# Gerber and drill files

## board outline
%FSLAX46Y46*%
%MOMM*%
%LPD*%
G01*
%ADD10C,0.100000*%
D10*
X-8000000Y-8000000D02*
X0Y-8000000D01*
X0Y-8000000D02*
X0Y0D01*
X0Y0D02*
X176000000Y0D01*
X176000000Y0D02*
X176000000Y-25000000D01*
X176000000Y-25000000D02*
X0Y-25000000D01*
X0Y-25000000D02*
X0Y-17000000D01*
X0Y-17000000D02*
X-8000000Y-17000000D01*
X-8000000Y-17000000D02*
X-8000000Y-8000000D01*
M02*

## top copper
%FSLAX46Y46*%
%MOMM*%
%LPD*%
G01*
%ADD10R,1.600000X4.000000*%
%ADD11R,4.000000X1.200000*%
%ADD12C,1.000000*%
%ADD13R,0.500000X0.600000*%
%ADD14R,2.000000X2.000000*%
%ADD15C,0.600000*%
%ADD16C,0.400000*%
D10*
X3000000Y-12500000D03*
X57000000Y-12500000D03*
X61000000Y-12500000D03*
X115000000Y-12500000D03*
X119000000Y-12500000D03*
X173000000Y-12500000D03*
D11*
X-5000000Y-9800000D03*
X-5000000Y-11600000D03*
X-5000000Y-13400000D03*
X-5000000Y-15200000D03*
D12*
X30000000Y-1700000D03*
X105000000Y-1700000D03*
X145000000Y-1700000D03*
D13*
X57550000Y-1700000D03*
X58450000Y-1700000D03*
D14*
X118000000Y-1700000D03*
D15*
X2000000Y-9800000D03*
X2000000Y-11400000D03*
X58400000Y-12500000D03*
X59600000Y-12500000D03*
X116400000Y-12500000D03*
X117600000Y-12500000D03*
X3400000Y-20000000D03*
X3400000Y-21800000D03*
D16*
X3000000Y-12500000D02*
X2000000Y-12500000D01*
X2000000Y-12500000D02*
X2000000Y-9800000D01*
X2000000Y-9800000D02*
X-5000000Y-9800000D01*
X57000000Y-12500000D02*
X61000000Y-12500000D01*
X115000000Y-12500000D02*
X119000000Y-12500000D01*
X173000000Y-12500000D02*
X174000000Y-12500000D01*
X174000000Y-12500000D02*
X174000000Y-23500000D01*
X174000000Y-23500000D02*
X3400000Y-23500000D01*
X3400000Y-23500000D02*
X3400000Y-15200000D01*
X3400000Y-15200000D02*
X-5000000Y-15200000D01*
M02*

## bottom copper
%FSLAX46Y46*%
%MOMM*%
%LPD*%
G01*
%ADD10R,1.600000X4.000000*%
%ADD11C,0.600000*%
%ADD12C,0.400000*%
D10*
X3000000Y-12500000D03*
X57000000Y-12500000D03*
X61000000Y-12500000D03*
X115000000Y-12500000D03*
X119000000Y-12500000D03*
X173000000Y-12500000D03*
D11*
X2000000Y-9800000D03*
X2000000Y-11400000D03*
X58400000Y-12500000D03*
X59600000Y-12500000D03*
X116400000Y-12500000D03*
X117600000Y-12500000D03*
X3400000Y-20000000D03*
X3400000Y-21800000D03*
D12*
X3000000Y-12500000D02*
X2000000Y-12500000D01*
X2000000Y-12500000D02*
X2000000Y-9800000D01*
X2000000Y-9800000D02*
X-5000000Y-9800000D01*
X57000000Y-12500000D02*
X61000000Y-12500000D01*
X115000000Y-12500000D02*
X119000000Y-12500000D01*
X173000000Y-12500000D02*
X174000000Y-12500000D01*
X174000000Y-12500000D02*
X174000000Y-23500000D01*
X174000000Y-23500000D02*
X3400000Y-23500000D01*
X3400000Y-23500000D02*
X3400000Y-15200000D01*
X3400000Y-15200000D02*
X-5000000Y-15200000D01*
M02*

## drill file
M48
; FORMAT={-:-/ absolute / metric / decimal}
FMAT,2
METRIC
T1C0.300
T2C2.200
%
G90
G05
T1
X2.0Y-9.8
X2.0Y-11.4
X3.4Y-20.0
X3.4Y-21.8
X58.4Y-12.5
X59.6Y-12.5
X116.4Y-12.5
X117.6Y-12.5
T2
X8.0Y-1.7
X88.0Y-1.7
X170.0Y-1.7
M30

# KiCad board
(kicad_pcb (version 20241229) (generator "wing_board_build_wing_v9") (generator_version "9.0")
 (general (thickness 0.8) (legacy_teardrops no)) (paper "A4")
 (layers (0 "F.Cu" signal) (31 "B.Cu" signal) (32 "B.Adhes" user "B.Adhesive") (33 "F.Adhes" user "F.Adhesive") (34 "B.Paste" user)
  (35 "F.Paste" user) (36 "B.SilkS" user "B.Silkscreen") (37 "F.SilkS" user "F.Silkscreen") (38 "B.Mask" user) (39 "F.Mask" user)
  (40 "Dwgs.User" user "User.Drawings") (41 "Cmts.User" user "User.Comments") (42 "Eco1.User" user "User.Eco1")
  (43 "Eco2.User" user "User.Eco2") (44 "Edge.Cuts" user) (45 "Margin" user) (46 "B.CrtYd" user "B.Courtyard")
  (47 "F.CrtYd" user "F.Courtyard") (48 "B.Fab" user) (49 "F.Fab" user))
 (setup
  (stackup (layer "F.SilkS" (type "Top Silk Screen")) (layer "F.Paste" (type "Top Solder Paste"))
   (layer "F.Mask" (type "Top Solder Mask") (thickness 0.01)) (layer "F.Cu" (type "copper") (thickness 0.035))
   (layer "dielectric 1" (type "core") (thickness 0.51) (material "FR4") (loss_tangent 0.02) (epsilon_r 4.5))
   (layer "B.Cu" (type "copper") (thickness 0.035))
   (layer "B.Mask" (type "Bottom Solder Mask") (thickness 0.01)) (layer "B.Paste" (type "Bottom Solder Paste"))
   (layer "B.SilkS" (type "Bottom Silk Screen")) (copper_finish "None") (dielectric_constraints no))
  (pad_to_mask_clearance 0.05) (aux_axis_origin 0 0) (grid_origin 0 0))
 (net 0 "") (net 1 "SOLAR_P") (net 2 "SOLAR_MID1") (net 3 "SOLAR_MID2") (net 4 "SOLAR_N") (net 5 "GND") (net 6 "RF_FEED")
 (gr_line (start -8 8) (end 0 8) (stroke (width 0.1) (type default)) (layer "Edge.Cuts"))
 (gr_line (start 0 8) (end 0 0) (stroke (width 0.1) (type default)) (layer "Edge.Cuts"))
 (gr_line (start 0 0) (end 176 0) (stroke (width 0.1) (type default)) (layer "Edge.Cuts"))
 (gr_line (start 176 0) (end 176 25) (stroke (width 0.1) (type default)) (layer "Edge.Cuts"))
 (gr_line (start 176 25) (end 0 25) (stroke (width 0.1) (type default)) (layer "Edge.Cuts"))
 (gr_line (start 0 25) (end 0 17) (stroke (width 0.1) (type default)) (layer "Edge.Cuts"))
 (gr_line (start 0 17) (end -8 17) (stroke (width 0.1) (type default)) (layer "Edge.Cuts"))
 (gr_line (start -8 17) (end -8 8) (stroke (width 0.1) (type default)) (layer "Edge.Cuts"))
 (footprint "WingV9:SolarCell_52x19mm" (layer "F.Cu") (at 30 12.5)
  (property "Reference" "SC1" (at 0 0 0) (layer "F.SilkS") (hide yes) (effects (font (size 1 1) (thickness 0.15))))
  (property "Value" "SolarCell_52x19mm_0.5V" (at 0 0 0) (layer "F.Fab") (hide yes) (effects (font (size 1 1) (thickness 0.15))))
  (pad "1" smd rect (at -27 0) (size 1.6 4) (layers "F.Cu" "F.Paste" "F.Mask") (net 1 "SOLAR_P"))
  (pad "2" smd rect (at 27 0) (size 1.6 4) (layers "F.Cu" "F.Paste" "F.Mask") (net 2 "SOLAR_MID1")))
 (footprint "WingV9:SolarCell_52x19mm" (layer "F.Cu") (at 88 12.5)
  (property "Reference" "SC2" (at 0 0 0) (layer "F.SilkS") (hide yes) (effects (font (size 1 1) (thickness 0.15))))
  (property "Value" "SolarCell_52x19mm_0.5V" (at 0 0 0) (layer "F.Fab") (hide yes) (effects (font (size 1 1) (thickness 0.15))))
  (pad "1" smd rect (at -27 0) (size 1.6 4) (layers "F.Cu" "F.Paste" "F.Mask") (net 2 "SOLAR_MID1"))
  (pad "2" smd rect (at 27 0) (size 1.6 4) (layers "F.Cu" "F.Paste" "F.Mask") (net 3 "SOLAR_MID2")))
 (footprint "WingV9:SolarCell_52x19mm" (layer "F.Cu") (at 146 12.5)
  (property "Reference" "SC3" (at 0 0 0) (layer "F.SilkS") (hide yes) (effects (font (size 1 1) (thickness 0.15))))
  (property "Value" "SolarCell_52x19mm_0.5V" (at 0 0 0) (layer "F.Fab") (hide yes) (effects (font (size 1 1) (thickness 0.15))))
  (pad "1" smd rect (at -27 0) (size 1.6 4) (layers "F.Cu" "F.Paste" "F.Mask") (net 3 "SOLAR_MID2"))
  (pad "2" smd rect (at 27 0) (size 1.6 4) (layers "F.Cu" "F.Paste" "F.Mask") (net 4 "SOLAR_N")))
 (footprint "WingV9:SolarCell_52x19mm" (layer "B.Cu") (at 30 12.5)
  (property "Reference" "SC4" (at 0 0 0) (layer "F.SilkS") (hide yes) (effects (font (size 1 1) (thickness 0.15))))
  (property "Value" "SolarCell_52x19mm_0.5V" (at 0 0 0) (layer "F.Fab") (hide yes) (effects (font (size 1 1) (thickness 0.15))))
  (pad "1" smd rect (at -27 0) (size 1.6 4) (layers "B.Cu" "B.Paste" "B.Mask") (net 1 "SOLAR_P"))
  (pad "2" smd rect (at 27 0) (size 1.6 4) (layers "B.Cu" "B.Paste" "B.Mask") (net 2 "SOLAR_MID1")))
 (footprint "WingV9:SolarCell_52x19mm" (layer "B.Cu") (at 88 12.5)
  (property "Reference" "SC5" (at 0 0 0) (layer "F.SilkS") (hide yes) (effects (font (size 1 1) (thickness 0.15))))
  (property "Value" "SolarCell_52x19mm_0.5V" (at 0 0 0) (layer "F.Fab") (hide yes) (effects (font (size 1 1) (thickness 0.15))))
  (pad "1" smd rect (at -27 0) (size 1.6 4) (layers "B.Cu" "B.Paste" "B.Mask") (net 2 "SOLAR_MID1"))
  (pad "2" smd rect (at 27 0) (size 1.6 4) (layers "B.Cu" "B.Paste" "B.Mask") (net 3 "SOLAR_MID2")))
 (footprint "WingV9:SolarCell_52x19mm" (layer "B.Cu") (at 146 12.5)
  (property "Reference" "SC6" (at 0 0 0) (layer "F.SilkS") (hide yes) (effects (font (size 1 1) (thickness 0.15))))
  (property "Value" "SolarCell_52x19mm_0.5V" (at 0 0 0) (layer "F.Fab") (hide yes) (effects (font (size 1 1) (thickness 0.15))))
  (pad "1" smd rect (at -27 0) (size 1.6 4) (layers "B.Cu" "B.Paste" "B.Mask") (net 3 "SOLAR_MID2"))
  (pad "2" smd rect (at 27 0) (size 1.6 4) (layers "B.Cu" "B.Paste" "B.Mask") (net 4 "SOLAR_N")))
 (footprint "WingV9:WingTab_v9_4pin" (layer "F.Cu") (at 0 0)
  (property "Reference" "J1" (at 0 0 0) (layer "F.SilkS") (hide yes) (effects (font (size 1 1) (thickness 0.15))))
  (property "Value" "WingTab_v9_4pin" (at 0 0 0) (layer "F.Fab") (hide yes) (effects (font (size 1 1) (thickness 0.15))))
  (pad "1" smd rect (at -5 9.8) (size 4 1.2) (layers "F.Cu" "F.Paste" "F.Mask") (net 1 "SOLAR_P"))
  (pad "2" smd rect (at -5 11.6) (size 4 1.2) (layers "F.Cu" "F.Paste" "F.Mask") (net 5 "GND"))
  (pad "3" smd rect (at -5 13.4) (size 4 1.2) (layers "F.Cu" "F.Paste" "F.Mask") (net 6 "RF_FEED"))
  (pad "4" smd rect (at -5 15.2) (size 4 1.2) (layers "F.Cu" "F.Paste" "F.Mask") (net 4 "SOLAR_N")))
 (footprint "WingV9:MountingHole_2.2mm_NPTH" (layer "F.Cu") (at 8 1.7)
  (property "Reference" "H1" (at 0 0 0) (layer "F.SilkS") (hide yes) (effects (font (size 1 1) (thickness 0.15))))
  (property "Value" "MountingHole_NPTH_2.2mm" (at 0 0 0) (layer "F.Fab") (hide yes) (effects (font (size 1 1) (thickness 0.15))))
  (pad "" np_thru_hole circle (at 0 0) (size 2.2 2.2) (drill 2.2) (layers "*.Cu" "*.Mask")))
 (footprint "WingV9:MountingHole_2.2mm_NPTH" (layer "F.Cu") (at 88 1.7)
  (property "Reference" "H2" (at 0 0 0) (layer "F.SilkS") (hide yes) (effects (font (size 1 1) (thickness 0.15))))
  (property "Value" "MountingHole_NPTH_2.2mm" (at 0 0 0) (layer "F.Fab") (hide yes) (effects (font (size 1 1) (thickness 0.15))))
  (pad "" np_thru_hole circle (at 0 0) (size 2.2 2.2) (drill 2.2) (layers "*.Cu" "*.Mask")))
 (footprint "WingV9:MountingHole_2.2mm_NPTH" (layer "F.Cu") (at 170 1.7)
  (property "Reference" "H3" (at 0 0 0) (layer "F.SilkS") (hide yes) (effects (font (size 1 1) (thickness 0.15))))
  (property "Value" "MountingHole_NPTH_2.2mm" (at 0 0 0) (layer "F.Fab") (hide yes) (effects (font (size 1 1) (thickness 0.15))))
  (pad "" np_thru_hole circle (at 0 0) (size 2.2 2.2) (drill 2.2) (layers "*.Cu" "*.Mask")))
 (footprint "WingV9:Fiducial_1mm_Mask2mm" (layer "F.Cu") (at 30 1.7)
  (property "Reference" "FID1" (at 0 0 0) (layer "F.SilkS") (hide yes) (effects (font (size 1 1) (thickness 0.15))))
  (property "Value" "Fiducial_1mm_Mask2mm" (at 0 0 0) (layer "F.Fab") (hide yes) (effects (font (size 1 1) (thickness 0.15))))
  (pad "1" smd circle (at 0 0) (size 1 1) (layers "F.Cu" "F.Mask")))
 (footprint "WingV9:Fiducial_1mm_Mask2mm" (layer "F.Cu") (at 105 1.7)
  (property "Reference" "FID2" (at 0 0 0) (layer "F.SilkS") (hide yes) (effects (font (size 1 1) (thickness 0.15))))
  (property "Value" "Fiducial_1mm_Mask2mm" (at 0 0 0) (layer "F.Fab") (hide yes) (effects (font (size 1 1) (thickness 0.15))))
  (pad "1" smd circle (at 0 0) (size 1 1) (layers "F.Cu" "F.Mask")))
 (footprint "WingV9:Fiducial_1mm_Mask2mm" (layer "F.Cu") (at 145 1.7)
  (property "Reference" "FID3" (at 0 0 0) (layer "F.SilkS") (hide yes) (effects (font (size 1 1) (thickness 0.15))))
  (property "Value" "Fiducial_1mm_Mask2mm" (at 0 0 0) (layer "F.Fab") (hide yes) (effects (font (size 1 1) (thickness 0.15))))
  (pad "1" smd circle (at 0 0) (size 1 1) (layers "F.Cu" "F.Mask")))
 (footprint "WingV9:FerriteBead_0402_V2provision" (layer "F.Cu") (at 58 1.7)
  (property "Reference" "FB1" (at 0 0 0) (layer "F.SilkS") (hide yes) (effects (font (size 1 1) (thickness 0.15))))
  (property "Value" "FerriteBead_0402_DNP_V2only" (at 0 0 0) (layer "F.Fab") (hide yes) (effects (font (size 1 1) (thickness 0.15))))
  (pad "1" smd rect (at -0.45 0) (size 0.5 0.6) (layers "F.Cu" "F.Paste" "F.Mask"))
  (pad "2" smd rect (at 0.45 0) (size 0.5 0.6) (layers "F.Cu" "F.Paste" "F.Mask")))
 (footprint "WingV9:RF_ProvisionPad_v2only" (layer "F.Cu") (at 118 1.7)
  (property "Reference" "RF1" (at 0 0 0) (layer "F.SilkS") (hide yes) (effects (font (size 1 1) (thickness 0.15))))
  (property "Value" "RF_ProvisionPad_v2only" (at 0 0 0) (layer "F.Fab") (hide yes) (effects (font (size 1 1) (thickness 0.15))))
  (pad "1" smd rect (at 0 0) (size 2 2) (layers "F.Cu" "F.Mask")))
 (segment (start 3 12.5) (end 2 12.5) (width 0.4) (layer "F.Cu") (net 1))
 (segment (start 2 12.5) (end 2 9.8) (width 0.4) (layer "F.Cu") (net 1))
 (segment (start 2 9.8) (end -5 9.8) (width 0.4) (layer "F.Cu") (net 1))
 (segment (start 57 12.5) (end 61 12.5) (width 0.4) (layer "F.Cu") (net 2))
 (segment (start 115 12.5) (end 119 12.5) (width 0.4) (layer "F.Cu") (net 3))
 (segment (start 173 12.5) (end 174 12.5) (width 0.4) (layer "F.Cu") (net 4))
 (segment (start 174 12.5) (end 174 23.5) (width 0.4) (layer "F.Cu") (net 4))
 (segment (start 174 23.5) (end 3.4 23.5) (width 0.4) (layer "F.Cu") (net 4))
 (segment (start 3.4 23.5) (end 3.4 15.2) (width 0.4) (layer "F.Cu") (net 4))
 (segment (start 3.4 15.2) (end -5 15.2) (width 0.4) (layer "F.Cu") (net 4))
 (segment (start 3 12.5) (end 2 12.5) (width 0.4) (layer "B.Cu") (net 1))
 (segment (start 2 12.5) (end 2 9.8) (width 0.4) (layer "B.Cu") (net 1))
 (segment (start 2 9.8) (end -5 9.8) (width 0.4) (layer "B.Cu") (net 1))
 (segment (start 57 12.5) (end 61 12.5) (width 0.4) (layer "B.Cu") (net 2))
 (segment (start 115 12.5) (end 119 12.5) (width 0.4) (layer "B.Cu") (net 3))
 (segment (start 173 12.5) (end 174 12.5) (width 0.4) (layer "B.Cu") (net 4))
 (segment (start 174 12.5) (end 174 23.5) (width 0.4) (layer "B.Cu") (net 4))
 (segment (start 174 23.5) (end 3.4 23.5) (width 0.4) (layer "B.Cu") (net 4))
 (segment (start 3.4 23.5) (end 3.4 15.2) (width 0.4) (layer "B.Cu") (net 4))
 (segment (start 3.4 15.2) (end -5 15.2) (width 0.4) (layer "B.Cu") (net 4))
 (via (at 2 9.8) (size 0.6) (drill 0.3) (layers "F.Cu" "B.Cu") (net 1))
 (via (at 2 11.4) (size 0.6) (drill 0.3) (layers "F.Cu" "B.Cu") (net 1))
 (via (at 58.4 12.5) (size 0.6) (drill 0.3) (layers "F.Cu" "B.Cu") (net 2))
 (via (at 59.6 12.5) (size 0.6) (drill 0.3) (layers "F.Cu" "B.Cu") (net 2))
 (via (at 116.4 12.5) (size 0.6) (drill 0.3) (layers "F.Cu" "B.Cu") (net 3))
 (via (at 117.6 12.5) (size 0.6) (drill 0.3) (layers "F.Cu" "B.Cu") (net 3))
 (via (at 3.4 20) (size 0.6) (drill 0.3) (layers "F.Cu" "B.Cu") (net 4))
 (via (at 3.4 21.8) (size 0.6) (drill 0.3) (layers "F.Cu" "B.Cu") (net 4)))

